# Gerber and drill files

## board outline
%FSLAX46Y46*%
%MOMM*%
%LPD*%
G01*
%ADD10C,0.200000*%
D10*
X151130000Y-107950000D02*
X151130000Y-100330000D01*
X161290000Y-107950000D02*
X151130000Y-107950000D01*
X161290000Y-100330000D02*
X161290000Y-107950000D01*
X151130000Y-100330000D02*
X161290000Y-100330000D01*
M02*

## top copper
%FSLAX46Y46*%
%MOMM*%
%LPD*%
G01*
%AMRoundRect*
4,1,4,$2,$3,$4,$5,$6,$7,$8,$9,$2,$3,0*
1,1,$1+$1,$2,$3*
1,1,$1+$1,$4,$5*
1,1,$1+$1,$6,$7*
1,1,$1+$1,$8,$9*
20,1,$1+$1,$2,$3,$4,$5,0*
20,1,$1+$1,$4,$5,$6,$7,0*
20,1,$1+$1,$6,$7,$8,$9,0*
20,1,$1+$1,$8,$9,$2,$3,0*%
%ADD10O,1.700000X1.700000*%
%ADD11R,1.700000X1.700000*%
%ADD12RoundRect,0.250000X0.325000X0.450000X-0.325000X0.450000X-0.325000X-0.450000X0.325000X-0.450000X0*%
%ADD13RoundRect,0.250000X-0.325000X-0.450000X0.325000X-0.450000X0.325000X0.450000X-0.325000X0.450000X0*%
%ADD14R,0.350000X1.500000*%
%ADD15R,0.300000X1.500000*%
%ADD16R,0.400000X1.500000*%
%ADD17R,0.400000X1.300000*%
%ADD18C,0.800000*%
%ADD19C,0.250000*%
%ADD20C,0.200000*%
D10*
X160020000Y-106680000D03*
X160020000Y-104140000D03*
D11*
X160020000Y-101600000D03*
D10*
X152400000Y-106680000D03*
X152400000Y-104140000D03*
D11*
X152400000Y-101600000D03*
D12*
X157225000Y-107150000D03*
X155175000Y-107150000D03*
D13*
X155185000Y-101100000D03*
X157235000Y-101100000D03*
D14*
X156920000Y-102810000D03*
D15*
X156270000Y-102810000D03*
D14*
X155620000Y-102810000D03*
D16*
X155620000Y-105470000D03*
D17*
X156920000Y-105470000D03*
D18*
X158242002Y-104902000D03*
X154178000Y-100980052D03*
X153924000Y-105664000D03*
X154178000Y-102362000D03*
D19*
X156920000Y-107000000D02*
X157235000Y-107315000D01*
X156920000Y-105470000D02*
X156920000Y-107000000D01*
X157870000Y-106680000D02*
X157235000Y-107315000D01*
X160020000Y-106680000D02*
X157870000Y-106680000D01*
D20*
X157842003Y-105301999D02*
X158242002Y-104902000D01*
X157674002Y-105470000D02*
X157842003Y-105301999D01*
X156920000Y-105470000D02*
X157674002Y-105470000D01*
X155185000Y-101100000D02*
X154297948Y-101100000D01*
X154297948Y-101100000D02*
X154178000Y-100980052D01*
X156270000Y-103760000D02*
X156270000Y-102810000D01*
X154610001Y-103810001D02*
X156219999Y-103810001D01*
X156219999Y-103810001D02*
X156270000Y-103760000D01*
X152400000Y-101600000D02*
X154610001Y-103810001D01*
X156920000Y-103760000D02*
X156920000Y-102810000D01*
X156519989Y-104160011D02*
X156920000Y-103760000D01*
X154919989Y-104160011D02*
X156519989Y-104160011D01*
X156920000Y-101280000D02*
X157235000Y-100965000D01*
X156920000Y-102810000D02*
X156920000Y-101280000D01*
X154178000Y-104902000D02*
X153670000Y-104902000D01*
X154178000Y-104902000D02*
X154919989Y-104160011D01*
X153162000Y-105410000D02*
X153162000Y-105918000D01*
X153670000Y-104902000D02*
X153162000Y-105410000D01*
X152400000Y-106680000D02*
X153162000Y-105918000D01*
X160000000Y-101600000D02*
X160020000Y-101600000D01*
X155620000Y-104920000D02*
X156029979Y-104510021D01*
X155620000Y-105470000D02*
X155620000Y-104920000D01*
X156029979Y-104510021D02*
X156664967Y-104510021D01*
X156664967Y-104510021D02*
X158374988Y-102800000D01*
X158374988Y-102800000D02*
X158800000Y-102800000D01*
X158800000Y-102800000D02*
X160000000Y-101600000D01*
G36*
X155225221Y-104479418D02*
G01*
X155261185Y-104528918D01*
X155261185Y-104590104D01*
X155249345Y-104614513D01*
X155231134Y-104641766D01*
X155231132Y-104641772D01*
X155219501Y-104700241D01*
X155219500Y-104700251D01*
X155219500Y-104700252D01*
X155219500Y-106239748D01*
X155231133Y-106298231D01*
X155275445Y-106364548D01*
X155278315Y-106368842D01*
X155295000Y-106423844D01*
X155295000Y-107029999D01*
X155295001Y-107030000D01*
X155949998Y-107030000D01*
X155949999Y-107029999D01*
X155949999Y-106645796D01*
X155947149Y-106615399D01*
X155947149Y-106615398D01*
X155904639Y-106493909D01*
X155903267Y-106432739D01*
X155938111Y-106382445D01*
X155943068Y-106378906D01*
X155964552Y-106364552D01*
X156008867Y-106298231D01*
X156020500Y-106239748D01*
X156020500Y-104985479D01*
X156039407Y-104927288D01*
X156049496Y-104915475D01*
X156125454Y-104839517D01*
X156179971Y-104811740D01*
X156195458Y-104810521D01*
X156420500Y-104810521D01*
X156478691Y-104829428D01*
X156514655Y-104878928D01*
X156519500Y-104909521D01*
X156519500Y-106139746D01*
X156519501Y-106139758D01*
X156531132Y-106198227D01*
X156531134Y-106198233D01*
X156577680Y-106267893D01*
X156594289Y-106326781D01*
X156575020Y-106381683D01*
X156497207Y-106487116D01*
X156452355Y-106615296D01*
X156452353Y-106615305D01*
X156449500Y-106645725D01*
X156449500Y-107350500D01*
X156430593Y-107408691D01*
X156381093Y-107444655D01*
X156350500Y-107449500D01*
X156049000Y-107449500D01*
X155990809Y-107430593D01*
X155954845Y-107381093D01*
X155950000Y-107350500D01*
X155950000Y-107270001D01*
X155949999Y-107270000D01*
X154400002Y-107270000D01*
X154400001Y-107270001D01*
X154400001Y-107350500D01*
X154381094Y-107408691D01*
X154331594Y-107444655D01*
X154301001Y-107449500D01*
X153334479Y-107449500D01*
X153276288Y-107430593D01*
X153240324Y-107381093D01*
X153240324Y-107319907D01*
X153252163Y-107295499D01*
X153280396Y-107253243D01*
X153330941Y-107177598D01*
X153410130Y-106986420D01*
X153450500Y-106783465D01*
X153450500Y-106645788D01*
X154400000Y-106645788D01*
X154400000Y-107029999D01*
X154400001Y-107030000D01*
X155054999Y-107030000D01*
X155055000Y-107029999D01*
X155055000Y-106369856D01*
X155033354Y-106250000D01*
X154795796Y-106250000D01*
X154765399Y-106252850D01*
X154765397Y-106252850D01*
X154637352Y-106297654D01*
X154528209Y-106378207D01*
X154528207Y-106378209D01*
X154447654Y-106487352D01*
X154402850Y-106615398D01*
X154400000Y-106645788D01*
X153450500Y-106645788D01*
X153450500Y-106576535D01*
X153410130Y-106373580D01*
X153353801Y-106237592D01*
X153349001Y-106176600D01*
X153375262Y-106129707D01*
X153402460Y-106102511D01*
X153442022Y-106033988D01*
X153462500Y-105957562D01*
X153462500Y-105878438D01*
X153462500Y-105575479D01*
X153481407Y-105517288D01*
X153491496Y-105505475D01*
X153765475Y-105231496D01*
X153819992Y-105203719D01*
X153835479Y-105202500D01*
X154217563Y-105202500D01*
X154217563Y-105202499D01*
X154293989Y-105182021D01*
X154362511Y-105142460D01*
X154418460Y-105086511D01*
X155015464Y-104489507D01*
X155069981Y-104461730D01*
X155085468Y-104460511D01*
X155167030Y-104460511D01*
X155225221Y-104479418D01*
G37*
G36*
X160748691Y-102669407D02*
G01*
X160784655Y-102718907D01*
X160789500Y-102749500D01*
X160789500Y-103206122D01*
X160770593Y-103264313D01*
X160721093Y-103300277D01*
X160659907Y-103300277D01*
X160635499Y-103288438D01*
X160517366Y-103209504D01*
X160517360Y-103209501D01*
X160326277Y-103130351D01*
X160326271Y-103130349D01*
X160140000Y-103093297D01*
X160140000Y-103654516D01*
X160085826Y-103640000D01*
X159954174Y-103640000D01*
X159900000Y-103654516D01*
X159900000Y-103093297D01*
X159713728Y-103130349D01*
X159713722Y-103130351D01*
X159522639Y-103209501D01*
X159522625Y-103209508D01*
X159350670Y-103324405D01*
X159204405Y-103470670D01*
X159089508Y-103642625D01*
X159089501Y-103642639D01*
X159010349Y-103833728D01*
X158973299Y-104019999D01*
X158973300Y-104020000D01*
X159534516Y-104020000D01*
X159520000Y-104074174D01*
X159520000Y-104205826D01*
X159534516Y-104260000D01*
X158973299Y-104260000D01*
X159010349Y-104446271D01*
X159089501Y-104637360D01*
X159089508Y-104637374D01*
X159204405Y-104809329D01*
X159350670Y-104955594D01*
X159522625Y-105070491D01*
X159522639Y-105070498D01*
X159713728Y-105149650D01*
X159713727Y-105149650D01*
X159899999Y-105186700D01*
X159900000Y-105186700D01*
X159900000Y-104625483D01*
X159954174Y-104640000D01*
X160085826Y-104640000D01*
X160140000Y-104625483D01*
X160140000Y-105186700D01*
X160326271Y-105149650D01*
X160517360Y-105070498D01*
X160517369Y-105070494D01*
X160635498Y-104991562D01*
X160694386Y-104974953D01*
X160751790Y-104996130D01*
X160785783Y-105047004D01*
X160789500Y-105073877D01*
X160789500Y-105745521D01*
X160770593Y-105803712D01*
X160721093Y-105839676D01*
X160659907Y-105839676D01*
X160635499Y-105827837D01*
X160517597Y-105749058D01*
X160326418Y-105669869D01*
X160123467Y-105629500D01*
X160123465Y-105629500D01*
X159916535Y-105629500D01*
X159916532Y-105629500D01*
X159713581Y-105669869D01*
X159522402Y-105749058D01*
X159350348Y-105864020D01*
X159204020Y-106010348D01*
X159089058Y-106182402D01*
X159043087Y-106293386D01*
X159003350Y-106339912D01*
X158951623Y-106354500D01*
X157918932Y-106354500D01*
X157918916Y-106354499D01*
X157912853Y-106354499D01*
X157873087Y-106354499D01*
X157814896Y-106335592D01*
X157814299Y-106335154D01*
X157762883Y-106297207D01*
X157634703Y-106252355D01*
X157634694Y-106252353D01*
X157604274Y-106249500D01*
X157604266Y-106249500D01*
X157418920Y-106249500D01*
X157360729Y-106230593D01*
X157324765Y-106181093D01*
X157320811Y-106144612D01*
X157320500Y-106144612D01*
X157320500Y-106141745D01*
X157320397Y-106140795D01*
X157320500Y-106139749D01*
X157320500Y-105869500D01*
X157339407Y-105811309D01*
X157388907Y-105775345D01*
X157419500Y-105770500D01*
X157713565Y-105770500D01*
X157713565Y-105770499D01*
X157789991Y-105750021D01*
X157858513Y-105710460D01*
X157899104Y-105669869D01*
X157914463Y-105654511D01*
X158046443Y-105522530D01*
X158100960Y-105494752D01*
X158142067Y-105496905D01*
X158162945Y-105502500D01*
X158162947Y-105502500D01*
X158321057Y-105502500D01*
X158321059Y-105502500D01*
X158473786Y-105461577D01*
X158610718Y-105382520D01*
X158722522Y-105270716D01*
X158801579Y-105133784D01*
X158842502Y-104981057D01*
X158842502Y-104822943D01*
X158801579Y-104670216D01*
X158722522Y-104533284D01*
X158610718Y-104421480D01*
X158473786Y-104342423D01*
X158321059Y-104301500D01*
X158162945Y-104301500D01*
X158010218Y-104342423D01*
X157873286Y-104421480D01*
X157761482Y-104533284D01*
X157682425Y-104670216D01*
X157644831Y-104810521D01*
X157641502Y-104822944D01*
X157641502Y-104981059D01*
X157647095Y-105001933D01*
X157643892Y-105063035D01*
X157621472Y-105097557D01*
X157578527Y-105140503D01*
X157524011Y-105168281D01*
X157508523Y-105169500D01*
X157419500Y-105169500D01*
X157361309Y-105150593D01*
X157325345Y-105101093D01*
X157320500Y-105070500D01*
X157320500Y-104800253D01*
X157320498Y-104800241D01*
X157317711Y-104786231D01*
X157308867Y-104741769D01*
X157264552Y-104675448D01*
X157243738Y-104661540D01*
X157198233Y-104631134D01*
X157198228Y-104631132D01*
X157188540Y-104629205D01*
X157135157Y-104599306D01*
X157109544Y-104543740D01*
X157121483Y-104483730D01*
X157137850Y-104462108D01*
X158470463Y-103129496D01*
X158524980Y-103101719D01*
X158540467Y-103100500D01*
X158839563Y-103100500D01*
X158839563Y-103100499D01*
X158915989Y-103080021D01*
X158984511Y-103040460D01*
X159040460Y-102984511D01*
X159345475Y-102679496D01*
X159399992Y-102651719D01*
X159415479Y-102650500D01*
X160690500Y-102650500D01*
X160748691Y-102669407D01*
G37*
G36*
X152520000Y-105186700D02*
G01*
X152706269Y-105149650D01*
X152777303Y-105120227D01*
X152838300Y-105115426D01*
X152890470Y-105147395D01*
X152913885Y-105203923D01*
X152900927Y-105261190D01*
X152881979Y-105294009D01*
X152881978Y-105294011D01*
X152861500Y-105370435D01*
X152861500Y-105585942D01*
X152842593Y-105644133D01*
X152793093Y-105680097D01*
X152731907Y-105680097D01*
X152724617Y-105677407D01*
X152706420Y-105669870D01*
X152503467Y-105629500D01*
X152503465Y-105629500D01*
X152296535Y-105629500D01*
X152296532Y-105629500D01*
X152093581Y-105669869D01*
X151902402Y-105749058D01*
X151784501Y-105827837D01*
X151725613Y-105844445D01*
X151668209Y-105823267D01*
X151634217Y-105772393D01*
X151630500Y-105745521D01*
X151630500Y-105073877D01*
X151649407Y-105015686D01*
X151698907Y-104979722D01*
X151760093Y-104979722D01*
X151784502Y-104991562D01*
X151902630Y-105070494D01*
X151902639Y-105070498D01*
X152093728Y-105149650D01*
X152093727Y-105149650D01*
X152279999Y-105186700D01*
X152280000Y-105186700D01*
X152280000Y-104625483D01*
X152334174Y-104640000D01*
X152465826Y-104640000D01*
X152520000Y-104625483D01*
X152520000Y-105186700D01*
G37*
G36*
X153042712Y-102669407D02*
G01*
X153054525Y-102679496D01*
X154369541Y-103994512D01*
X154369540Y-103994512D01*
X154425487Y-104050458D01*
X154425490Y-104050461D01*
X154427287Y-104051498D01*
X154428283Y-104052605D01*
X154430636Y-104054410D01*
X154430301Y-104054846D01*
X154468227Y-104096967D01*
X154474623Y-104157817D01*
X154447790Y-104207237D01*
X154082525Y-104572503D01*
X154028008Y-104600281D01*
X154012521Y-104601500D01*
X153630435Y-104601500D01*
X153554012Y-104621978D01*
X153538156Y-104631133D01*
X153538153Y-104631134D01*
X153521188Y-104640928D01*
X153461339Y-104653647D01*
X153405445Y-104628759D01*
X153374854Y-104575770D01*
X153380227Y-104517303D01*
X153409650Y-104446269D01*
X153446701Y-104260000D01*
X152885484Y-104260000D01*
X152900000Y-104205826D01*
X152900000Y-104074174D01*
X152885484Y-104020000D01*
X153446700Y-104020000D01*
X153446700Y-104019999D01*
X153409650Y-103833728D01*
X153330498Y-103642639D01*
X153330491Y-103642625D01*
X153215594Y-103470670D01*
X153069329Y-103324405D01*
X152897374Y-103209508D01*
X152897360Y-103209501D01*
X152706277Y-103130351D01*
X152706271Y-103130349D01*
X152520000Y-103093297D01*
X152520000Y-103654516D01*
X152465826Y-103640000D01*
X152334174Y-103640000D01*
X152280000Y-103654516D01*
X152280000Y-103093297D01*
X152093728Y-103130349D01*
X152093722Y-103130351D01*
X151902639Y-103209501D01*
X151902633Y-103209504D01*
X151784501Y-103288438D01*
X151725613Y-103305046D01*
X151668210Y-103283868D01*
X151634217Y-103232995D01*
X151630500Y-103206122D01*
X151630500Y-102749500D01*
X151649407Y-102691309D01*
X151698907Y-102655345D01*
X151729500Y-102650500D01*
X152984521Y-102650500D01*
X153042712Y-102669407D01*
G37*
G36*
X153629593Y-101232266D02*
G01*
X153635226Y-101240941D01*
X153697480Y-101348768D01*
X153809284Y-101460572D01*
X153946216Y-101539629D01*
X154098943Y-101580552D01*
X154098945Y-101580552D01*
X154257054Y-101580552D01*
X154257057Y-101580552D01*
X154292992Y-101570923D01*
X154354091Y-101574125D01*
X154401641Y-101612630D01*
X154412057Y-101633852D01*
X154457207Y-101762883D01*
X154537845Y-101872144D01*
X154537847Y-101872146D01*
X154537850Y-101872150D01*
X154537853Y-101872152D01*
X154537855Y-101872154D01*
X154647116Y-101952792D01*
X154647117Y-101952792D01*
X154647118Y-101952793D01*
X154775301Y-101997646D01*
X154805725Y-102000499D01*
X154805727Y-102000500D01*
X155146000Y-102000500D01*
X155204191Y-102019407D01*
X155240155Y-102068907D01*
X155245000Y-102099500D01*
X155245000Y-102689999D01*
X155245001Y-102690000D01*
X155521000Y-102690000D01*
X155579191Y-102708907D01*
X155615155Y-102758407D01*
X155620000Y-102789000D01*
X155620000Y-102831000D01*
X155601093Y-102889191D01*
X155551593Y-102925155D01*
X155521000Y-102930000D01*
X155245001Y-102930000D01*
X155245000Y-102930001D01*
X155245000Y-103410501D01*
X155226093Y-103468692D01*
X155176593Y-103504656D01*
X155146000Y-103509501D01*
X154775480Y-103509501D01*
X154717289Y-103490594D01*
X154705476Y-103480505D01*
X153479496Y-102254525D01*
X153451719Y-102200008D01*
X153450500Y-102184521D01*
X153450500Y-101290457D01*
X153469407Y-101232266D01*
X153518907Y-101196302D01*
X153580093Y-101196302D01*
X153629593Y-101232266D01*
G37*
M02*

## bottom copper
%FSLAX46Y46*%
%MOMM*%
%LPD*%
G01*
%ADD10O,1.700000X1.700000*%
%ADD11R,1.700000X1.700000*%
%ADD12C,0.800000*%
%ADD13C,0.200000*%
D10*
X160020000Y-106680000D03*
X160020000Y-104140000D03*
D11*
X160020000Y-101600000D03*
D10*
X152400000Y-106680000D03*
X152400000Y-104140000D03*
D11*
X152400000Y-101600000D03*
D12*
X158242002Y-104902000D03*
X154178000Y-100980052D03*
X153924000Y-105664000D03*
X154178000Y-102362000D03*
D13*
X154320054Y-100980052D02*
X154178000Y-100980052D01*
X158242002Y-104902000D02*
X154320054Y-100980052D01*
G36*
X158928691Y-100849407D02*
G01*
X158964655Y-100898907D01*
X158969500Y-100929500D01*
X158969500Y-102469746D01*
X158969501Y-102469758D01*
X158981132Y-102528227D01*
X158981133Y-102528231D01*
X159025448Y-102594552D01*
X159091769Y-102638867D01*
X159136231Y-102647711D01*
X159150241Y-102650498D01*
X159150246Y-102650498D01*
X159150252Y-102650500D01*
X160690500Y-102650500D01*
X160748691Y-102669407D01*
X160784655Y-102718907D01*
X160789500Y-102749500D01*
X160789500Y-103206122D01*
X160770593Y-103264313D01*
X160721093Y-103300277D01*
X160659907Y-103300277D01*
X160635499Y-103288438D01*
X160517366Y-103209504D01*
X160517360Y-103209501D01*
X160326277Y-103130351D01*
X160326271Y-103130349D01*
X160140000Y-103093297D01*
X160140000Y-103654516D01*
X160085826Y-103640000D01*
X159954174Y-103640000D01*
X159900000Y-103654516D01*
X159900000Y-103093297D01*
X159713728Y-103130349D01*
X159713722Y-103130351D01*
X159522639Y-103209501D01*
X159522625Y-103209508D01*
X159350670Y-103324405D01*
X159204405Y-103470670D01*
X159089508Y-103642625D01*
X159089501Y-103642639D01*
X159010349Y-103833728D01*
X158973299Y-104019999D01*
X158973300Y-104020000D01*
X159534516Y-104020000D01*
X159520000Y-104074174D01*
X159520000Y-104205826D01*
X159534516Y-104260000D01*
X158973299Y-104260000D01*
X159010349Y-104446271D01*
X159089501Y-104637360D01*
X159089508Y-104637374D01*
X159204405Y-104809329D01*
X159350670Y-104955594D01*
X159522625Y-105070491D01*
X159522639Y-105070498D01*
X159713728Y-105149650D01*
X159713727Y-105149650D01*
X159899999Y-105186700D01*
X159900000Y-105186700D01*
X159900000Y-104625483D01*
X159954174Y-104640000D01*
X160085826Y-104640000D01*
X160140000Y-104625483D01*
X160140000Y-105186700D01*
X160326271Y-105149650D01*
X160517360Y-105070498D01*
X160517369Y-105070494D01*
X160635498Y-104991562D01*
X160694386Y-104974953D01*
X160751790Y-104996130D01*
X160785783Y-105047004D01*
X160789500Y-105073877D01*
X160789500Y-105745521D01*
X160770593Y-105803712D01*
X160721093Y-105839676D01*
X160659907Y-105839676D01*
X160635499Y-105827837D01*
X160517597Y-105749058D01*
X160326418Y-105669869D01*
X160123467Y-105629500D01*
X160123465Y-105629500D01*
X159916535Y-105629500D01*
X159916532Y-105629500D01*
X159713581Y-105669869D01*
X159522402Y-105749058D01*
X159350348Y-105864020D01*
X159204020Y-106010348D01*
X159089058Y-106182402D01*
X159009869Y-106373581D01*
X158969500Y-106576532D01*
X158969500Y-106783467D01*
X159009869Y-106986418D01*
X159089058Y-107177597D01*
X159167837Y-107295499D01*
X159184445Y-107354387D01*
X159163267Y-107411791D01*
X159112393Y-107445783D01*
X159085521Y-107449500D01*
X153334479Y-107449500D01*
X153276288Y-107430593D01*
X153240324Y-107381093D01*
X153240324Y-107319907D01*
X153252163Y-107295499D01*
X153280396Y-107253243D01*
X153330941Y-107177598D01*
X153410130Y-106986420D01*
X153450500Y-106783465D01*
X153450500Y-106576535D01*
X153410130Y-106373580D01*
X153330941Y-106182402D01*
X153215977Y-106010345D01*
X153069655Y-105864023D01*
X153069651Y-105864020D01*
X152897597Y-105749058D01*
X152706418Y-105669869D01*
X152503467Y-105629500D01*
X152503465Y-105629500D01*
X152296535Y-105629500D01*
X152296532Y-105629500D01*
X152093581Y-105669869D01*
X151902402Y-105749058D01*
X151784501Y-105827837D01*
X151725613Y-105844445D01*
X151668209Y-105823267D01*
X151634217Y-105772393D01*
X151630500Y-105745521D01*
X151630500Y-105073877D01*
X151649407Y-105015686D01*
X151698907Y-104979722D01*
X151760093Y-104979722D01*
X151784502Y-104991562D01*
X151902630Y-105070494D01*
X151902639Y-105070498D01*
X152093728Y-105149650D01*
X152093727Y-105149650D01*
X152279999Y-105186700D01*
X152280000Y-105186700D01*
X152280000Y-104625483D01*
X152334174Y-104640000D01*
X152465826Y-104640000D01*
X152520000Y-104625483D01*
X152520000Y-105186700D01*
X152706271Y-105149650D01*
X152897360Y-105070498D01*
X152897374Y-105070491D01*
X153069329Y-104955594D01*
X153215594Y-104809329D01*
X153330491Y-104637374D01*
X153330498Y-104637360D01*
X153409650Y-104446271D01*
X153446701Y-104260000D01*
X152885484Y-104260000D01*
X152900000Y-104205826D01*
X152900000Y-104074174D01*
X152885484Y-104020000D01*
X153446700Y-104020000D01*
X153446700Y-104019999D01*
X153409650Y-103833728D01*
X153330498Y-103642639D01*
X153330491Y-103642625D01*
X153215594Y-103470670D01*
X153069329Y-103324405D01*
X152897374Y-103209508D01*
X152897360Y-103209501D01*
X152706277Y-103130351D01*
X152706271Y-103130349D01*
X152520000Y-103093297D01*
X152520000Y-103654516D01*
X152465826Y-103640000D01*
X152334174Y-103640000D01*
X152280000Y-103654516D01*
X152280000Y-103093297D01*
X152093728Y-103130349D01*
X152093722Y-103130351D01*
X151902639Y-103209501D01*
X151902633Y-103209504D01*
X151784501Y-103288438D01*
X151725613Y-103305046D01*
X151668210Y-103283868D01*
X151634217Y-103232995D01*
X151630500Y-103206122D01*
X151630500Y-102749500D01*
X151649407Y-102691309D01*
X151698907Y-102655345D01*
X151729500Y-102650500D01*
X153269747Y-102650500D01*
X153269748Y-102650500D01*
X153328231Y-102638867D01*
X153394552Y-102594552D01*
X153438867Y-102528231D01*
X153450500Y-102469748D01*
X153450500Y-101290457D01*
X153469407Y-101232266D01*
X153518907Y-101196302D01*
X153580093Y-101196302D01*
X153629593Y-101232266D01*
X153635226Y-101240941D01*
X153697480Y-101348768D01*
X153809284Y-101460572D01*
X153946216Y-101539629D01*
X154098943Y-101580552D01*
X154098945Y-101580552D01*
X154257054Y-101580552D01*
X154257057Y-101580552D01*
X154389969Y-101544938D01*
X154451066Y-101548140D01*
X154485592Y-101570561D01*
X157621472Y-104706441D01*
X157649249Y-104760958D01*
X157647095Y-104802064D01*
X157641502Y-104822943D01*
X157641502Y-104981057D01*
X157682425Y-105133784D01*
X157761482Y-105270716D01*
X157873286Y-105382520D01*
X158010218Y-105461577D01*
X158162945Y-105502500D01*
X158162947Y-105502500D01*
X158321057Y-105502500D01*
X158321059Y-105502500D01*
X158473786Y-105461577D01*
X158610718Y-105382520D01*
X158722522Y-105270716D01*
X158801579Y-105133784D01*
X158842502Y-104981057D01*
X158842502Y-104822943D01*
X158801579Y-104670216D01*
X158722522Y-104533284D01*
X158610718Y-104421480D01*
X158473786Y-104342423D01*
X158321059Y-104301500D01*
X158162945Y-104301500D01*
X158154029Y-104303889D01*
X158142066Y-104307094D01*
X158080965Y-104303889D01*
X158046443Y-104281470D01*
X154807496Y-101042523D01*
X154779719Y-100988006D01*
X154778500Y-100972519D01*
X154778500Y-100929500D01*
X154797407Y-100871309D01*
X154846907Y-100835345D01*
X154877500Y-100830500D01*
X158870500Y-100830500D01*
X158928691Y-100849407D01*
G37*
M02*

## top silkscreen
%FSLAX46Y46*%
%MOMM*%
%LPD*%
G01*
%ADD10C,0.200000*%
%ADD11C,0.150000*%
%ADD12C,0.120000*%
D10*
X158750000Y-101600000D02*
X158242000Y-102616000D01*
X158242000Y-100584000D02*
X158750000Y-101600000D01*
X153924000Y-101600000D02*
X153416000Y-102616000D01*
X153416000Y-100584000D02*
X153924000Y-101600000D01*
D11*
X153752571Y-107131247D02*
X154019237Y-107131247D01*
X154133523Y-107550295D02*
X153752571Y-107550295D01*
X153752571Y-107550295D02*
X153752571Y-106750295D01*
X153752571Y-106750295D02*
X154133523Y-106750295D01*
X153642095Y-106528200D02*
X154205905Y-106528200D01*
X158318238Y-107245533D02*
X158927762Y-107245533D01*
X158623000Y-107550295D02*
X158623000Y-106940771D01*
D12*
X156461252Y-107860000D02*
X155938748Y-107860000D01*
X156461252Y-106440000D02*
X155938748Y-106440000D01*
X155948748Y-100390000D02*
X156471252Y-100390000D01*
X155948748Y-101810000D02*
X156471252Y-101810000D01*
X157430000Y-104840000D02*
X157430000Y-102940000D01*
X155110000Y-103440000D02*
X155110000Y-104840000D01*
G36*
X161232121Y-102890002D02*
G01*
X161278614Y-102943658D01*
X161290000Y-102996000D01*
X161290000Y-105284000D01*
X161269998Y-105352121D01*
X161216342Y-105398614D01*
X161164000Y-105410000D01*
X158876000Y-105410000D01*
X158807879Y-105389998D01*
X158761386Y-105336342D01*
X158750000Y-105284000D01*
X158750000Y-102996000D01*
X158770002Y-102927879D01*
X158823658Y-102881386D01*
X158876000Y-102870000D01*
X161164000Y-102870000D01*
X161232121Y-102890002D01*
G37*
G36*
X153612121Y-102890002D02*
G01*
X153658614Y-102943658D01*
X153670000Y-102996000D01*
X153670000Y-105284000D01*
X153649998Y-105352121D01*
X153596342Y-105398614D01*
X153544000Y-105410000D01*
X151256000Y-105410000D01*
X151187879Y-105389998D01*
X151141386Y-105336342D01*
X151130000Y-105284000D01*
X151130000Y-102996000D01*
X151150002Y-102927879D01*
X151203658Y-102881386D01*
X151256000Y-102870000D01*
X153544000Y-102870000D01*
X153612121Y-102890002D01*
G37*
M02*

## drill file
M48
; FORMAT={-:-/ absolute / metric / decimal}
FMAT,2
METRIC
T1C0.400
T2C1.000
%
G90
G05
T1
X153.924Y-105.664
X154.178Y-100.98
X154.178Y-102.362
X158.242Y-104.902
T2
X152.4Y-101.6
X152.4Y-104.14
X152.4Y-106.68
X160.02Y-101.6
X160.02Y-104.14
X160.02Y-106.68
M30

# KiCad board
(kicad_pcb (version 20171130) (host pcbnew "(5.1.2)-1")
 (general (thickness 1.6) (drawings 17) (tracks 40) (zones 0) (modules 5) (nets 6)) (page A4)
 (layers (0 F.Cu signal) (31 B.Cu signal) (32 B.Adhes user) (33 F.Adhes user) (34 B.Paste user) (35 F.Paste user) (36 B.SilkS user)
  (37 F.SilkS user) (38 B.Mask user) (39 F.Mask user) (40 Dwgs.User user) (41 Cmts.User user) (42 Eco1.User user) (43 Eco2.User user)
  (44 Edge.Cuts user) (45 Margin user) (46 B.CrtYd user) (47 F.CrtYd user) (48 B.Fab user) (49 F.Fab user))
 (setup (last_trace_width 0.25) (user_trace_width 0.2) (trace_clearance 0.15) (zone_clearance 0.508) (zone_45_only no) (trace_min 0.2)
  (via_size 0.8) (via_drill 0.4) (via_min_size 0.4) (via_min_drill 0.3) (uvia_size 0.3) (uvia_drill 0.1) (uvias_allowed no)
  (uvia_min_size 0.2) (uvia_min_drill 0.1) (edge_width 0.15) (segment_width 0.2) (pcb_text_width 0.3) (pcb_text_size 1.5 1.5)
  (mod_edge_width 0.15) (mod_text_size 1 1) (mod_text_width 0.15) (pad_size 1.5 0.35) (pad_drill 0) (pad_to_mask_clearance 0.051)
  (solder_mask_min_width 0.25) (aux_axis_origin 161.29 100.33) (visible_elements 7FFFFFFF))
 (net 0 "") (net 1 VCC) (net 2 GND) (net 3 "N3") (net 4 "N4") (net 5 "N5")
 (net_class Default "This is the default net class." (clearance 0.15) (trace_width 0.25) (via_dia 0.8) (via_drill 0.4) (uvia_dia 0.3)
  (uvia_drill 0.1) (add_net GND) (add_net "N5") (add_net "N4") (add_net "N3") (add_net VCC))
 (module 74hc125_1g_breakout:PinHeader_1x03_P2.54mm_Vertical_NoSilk (layer F.Cu) (at 160.02 101.6)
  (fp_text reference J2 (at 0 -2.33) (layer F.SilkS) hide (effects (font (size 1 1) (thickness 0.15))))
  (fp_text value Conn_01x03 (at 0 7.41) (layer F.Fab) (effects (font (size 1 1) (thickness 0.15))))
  (pad 3 thru_hole oval (at 0 5.08) (size 1.7 1.7) (drill 1) (layers *.Cu *.Mask) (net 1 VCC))
  (pad 2 thru_hole oval (at 0 2.54) (size 1.7 1.7) (drill 1) (layers *.Cu *.Mask) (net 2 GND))
  (pad 1 thru_hole rect (at 0 0) (size 1.7 1.7) (drill 1) (layers *.Cu *.Mask) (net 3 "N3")))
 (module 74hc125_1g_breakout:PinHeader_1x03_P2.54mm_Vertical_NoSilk (layer F.Cu) (at 152.4 101.6)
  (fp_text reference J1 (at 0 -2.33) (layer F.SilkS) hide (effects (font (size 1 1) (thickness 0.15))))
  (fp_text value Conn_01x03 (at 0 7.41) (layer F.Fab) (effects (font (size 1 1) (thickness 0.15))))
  (pad 3 thru_hole oval (at 0 5.08) (size 1.7 1.7) (drill 1) (layers *.Cu *.Mask) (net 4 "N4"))
  (pad 2 thru_hole oval (at 0 2.54) (size 1.7 1.7) (drill 1) (layers *.Cu *.Mask) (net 2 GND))
  (pad 1 thru_hole rect (at 0 0) (size 1.7 1.7) (drill 1) (layers *.Cu *.Mask) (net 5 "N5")))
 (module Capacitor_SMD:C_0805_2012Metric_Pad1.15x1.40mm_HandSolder (layer F.Cu) (at 156.2 107.15 180)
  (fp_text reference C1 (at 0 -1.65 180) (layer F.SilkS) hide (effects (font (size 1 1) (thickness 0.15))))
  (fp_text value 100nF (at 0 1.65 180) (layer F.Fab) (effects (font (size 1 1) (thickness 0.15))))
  (fp_line (start -0.261252 -0.71) (end 0.261252 -0.71) (layer F.SilkS) (width 0.12))
  (fp_line (start -0.261252 0.71) (end 0.261252 0.71) (layer F.SilkS) (width 0.12))
  (pad 1 smd roundrect (at -1.025 0 180) (size 1.15 1.4) (layers F.Cu F.Paste F.Mask) (roundrect_rratio 0.217391) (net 1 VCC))
  (pad 2 smd roundrect (at 1.025 0 180) (size 1.15 1.4) (layers F.Cu F.Paste F.Mask) (roundrect_rratio 0.217391) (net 2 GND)))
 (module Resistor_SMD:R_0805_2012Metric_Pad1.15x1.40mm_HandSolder (layer F.Cu) (at 156.21 101.1)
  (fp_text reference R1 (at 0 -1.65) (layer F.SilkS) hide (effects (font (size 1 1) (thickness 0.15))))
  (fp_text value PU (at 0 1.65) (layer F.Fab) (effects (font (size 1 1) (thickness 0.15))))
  (fp_line (start -0.261252 -0.71) (end 0.261252 -0.71) (layer F.SilkS) (width 0.12))
  (fp_line (start -0.261252 0.71) (end 0.261252 0.71) (layer F.SilkS) (width 0.12))
  (pad 1 smd roundrect (at -1.025 0) (size 1.15 1.4) (layers F.Cu F.Paste F.Mask) (roundrect_rratio 0.217391) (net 1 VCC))
  (pad 2 smd roundrect (at 1.025 0) (size 1.15 1.4) (layers F.Cu F.Paste F.Mask) (roundrect_rratio 0.217391) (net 4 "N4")))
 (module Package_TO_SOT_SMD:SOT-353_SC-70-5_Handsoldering (layer F.Cu) (at 156.27 104.14 270)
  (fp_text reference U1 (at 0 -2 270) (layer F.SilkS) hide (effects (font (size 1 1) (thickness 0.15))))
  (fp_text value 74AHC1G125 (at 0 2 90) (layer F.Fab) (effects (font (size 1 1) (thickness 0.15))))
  (fp_line (start 0.7 -1.16) (end -1.2 -1.16) (layer F.SilkS) (width 0.12))
  (fp_line (start -0.7 1.16) (end 0.7 1.16) (layer F.SilkS) (width 0.12))
  (pad 1 smd rect (at -1.33 -0.65 270) (size 1.5 0.35) (layers F.Cu F.Paste F.Mask) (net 4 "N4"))
  (pad 2 smd rect (at -1.33 0 270) (size 1.5 0.3) (layers F.Cu F.Paste F.Mask) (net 5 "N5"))
  (pad 3 smd rect (at -1.33 0.65 270) (size 1.5 0.35) (layers F.Cu F.Paste F.Mask) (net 2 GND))
  (pad 4 smd rect (at 1.33 0.65 270) (size 1.5 0.4) (layers F.Cu F.Paste F.Mask) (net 3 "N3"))
  (pad 5 smd rect (at 1.33 -0.65 270) (size 1.3 0.4) (layers F.Cu F.Paste F.Mask) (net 1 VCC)))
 (gr_line (start 158.75 101.6) (end 158.242 102.616) (layer F.SilkS) (width 0.2))
 (gr_line (start 158.242 100.584) (end 158.75 101.6) (layer F.SilkS) (width 0.2))
 (gr_line (start 153.924 101.6) (end 153.416 102.616) (layer F.SilkS) (width 0.2))
 (gr_line (start 153.416 100.584) (end 153.924 101.6) (layer F.SilkS) (width 0.2))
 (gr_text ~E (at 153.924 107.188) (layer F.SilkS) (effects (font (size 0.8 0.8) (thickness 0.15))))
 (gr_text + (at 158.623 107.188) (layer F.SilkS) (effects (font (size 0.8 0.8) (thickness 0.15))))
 (gr_line (start 151.13 107.95) (end 151.13 100.33) (layer Edge.Cuts) (width 0.2))
 (gr_line (start 161.29 107.95) (end 151.13 107.95) (layer Edge.Cuts) (width 0.2))
 (gr_line (start 161.29 100.33) (end 161.29 107.95) (layer Edge.Cuts) (width 0.2))
 (gr_line (start 151.13 100.33) (end 161.29 100.33) (layer Edge.Cuts) (width 0.2))
 (segment (start 167.132 103.632) (end 169.164 103.632) (width 0.2) (layer F.SilkS) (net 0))
 (segment (start 169.164 103.632) (end 169.418 103.886) (width 0.2) (layer F.SilkS) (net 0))
 (segment (start 169.418 103.886) (end 170.688 103.886) (width 0.2) (layer F.SilkS) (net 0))
 (segment (start 170.688 103.886) (end 172.212 105.41) (width 0.2) (layer F.SilkS) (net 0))
 (segment (start 156.92 107) (end 157.235 107.315) (width 0.25) (layer F.Cu) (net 1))
 (segment (start 156.92 105.47) (end 156.92 107) (width 0.25) (layer F.Cu) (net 1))
 (segment (start 157.87 106.68) (end 157.235 107.315) (width 0.25) (layer F.Cu) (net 1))
 (segment (start 160.02 106.68) (end 157.87 106.68) (width 0.25) (layer F.Cu) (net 1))
 (via (at 158.242002 104.902) (size 0.8) (drill 0.4) (layers F.Cu B.Cu) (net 1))
 (segment (start 157.842003 105.301999) (end 158.242002 104.902) (width 0.2) (layer F.Cu) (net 1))
 (segment (start 157.674002 105.47) (end 157.842003 105.301999) (width 0.2) (layer F.Cu) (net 1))
 (segment (start 156.92 105.47) (end 157.674002 105.47) (width 0.2) (layer F.Cu) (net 1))
 (via (at 154.178 100.980052) (size 0.8) (drill 0.4) (layers F.Cu B.Cu) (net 1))
 (segment (start 155.185 101.1) (end 154.297948 101.1) (width 0.2) (layer F.Cu) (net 1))
 (segment (start 154.297948 101.1) (end 154.178 100.980052) (width 0.2) (layer F.Cu) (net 1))
 (segment (start 154.320054 100.980052) (end 154.178 100.980052) (width 0.2) (layer B.Cu) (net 1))
 (segment (start 158.242002 104.902) (end 154.320054 100.980052) (width 0.2) (layer B.Cu) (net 1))
 (via (at 153.924 105.664) (size 0.8) (drill 0.4) (layers F.Cu B.Cu) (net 2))
 (via (at 154.178 102.362) (size 0.8) (drill 0.4) (layers F.Cu B.Cu) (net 2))
 (segment (start 156.27 103.76) (end 156.27 102.81) (width 0.2) (layer F.Cu) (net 5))
 (segment (start 154.610001 103.810001) (end 156.219999 103.810001) (width 0.2) (layer F.Cu) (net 5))
 (segment (start 156.219999 103.810001) (end 156.27 103.76) (width 0.2) (layer F.Cu) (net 5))
 (segment (start 152.4 101.6) (end 154.610001 103.810001) (width 0.2) (layer F.Cu) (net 5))
 (segment (start 156.92 103.76) (end 156.92 102.81) (width 0.2) (layer F.Cu) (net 4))
 (segment (start 156.519989 104.160011) (end 156.92 103.76) (width 0.2) (layer F.Cu) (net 4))
 (segment (start 154.919989 104.160011) (end 156.519989 104.160011) (width 0.2) (layer F.Cu) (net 4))
 (segment (start 156.92 101.28) (end 157.235 100.965) (width 0.2) (layer F.Cu) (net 4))
 (segment (start 156.92 102.81) (end 156.92 101.28) (width 0.2) (layer F.Cu) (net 4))
 (segment (start 154.178 104.902) (end 153.67 104.902) (width 0.2) (layer F.Cu) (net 4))
 (segment (start 154.178 104.902) (end 154.919989 104.160011) (width 0.2) (layer F.Cu) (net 4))
 (segment (start 153.162 105.41) (end 153.162 105.918) (width 0.2) (layer F.Cu) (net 4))
 (segment (start 153.67 104.902) (end 153.162 105.41) (width 0.2) (layer F.Cu) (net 4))
 (segment (start 152.4 106.68) (end 153.162 105.918) (width 0.2) (layer F.Cu) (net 4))
 (segment (start 160 101.6) (end 160.02 101.6) (width 0.2) (layer F.Cu) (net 3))
 (segment (start 155.62 104.92) (end 156.029979 104.510021) (width 0.2) (layer F.Cu) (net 3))
 (segment (start 155.62 105.47) (end 155.62 104.92) (width 0.2) (layer F.Cu) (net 3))
 (segment (start 156.029979 104.510021) (end 156.664967 104.510021) (width 0.2) (layer F.Cu) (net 3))
 (segment (start 156.664967 104.510021) (end 158.374988 102.8) (width 0.2) (layer F.Cu) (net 3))
 (segment (start 158.374988 102.8) (end 158.8 102.8) (width 0.2) (layer F.Cu) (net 3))
 (segment (start 158.8 102.8) (end 160 101.6) (width 0.2) (layer F.Cu) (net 3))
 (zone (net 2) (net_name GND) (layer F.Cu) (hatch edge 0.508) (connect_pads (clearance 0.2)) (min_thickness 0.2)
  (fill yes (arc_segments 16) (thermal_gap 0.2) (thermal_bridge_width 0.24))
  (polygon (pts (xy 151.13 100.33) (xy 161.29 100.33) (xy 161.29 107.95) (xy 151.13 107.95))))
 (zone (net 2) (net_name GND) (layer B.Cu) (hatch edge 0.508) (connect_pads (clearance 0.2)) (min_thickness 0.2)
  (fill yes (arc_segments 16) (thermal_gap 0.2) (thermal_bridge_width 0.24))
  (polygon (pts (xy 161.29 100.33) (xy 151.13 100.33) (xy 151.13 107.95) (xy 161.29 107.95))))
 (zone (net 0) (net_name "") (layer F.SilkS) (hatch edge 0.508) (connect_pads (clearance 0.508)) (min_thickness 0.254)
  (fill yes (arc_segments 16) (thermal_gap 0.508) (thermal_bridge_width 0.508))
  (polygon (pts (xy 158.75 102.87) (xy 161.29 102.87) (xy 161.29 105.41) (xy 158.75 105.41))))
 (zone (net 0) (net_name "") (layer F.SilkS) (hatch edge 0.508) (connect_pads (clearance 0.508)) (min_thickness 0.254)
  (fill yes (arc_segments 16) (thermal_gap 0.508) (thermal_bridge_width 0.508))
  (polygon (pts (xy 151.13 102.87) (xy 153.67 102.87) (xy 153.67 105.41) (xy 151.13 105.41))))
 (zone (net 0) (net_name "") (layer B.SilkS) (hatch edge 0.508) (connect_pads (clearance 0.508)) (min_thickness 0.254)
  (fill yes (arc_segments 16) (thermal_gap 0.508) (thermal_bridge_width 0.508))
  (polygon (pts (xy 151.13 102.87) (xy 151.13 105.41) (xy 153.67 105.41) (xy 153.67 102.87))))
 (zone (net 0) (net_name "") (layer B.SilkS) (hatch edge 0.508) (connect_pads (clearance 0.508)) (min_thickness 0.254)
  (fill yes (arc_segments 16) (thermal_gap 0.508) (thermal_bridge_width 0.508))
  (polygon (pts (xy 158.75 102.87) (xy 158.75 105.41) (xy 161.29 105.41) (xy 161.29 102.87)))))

